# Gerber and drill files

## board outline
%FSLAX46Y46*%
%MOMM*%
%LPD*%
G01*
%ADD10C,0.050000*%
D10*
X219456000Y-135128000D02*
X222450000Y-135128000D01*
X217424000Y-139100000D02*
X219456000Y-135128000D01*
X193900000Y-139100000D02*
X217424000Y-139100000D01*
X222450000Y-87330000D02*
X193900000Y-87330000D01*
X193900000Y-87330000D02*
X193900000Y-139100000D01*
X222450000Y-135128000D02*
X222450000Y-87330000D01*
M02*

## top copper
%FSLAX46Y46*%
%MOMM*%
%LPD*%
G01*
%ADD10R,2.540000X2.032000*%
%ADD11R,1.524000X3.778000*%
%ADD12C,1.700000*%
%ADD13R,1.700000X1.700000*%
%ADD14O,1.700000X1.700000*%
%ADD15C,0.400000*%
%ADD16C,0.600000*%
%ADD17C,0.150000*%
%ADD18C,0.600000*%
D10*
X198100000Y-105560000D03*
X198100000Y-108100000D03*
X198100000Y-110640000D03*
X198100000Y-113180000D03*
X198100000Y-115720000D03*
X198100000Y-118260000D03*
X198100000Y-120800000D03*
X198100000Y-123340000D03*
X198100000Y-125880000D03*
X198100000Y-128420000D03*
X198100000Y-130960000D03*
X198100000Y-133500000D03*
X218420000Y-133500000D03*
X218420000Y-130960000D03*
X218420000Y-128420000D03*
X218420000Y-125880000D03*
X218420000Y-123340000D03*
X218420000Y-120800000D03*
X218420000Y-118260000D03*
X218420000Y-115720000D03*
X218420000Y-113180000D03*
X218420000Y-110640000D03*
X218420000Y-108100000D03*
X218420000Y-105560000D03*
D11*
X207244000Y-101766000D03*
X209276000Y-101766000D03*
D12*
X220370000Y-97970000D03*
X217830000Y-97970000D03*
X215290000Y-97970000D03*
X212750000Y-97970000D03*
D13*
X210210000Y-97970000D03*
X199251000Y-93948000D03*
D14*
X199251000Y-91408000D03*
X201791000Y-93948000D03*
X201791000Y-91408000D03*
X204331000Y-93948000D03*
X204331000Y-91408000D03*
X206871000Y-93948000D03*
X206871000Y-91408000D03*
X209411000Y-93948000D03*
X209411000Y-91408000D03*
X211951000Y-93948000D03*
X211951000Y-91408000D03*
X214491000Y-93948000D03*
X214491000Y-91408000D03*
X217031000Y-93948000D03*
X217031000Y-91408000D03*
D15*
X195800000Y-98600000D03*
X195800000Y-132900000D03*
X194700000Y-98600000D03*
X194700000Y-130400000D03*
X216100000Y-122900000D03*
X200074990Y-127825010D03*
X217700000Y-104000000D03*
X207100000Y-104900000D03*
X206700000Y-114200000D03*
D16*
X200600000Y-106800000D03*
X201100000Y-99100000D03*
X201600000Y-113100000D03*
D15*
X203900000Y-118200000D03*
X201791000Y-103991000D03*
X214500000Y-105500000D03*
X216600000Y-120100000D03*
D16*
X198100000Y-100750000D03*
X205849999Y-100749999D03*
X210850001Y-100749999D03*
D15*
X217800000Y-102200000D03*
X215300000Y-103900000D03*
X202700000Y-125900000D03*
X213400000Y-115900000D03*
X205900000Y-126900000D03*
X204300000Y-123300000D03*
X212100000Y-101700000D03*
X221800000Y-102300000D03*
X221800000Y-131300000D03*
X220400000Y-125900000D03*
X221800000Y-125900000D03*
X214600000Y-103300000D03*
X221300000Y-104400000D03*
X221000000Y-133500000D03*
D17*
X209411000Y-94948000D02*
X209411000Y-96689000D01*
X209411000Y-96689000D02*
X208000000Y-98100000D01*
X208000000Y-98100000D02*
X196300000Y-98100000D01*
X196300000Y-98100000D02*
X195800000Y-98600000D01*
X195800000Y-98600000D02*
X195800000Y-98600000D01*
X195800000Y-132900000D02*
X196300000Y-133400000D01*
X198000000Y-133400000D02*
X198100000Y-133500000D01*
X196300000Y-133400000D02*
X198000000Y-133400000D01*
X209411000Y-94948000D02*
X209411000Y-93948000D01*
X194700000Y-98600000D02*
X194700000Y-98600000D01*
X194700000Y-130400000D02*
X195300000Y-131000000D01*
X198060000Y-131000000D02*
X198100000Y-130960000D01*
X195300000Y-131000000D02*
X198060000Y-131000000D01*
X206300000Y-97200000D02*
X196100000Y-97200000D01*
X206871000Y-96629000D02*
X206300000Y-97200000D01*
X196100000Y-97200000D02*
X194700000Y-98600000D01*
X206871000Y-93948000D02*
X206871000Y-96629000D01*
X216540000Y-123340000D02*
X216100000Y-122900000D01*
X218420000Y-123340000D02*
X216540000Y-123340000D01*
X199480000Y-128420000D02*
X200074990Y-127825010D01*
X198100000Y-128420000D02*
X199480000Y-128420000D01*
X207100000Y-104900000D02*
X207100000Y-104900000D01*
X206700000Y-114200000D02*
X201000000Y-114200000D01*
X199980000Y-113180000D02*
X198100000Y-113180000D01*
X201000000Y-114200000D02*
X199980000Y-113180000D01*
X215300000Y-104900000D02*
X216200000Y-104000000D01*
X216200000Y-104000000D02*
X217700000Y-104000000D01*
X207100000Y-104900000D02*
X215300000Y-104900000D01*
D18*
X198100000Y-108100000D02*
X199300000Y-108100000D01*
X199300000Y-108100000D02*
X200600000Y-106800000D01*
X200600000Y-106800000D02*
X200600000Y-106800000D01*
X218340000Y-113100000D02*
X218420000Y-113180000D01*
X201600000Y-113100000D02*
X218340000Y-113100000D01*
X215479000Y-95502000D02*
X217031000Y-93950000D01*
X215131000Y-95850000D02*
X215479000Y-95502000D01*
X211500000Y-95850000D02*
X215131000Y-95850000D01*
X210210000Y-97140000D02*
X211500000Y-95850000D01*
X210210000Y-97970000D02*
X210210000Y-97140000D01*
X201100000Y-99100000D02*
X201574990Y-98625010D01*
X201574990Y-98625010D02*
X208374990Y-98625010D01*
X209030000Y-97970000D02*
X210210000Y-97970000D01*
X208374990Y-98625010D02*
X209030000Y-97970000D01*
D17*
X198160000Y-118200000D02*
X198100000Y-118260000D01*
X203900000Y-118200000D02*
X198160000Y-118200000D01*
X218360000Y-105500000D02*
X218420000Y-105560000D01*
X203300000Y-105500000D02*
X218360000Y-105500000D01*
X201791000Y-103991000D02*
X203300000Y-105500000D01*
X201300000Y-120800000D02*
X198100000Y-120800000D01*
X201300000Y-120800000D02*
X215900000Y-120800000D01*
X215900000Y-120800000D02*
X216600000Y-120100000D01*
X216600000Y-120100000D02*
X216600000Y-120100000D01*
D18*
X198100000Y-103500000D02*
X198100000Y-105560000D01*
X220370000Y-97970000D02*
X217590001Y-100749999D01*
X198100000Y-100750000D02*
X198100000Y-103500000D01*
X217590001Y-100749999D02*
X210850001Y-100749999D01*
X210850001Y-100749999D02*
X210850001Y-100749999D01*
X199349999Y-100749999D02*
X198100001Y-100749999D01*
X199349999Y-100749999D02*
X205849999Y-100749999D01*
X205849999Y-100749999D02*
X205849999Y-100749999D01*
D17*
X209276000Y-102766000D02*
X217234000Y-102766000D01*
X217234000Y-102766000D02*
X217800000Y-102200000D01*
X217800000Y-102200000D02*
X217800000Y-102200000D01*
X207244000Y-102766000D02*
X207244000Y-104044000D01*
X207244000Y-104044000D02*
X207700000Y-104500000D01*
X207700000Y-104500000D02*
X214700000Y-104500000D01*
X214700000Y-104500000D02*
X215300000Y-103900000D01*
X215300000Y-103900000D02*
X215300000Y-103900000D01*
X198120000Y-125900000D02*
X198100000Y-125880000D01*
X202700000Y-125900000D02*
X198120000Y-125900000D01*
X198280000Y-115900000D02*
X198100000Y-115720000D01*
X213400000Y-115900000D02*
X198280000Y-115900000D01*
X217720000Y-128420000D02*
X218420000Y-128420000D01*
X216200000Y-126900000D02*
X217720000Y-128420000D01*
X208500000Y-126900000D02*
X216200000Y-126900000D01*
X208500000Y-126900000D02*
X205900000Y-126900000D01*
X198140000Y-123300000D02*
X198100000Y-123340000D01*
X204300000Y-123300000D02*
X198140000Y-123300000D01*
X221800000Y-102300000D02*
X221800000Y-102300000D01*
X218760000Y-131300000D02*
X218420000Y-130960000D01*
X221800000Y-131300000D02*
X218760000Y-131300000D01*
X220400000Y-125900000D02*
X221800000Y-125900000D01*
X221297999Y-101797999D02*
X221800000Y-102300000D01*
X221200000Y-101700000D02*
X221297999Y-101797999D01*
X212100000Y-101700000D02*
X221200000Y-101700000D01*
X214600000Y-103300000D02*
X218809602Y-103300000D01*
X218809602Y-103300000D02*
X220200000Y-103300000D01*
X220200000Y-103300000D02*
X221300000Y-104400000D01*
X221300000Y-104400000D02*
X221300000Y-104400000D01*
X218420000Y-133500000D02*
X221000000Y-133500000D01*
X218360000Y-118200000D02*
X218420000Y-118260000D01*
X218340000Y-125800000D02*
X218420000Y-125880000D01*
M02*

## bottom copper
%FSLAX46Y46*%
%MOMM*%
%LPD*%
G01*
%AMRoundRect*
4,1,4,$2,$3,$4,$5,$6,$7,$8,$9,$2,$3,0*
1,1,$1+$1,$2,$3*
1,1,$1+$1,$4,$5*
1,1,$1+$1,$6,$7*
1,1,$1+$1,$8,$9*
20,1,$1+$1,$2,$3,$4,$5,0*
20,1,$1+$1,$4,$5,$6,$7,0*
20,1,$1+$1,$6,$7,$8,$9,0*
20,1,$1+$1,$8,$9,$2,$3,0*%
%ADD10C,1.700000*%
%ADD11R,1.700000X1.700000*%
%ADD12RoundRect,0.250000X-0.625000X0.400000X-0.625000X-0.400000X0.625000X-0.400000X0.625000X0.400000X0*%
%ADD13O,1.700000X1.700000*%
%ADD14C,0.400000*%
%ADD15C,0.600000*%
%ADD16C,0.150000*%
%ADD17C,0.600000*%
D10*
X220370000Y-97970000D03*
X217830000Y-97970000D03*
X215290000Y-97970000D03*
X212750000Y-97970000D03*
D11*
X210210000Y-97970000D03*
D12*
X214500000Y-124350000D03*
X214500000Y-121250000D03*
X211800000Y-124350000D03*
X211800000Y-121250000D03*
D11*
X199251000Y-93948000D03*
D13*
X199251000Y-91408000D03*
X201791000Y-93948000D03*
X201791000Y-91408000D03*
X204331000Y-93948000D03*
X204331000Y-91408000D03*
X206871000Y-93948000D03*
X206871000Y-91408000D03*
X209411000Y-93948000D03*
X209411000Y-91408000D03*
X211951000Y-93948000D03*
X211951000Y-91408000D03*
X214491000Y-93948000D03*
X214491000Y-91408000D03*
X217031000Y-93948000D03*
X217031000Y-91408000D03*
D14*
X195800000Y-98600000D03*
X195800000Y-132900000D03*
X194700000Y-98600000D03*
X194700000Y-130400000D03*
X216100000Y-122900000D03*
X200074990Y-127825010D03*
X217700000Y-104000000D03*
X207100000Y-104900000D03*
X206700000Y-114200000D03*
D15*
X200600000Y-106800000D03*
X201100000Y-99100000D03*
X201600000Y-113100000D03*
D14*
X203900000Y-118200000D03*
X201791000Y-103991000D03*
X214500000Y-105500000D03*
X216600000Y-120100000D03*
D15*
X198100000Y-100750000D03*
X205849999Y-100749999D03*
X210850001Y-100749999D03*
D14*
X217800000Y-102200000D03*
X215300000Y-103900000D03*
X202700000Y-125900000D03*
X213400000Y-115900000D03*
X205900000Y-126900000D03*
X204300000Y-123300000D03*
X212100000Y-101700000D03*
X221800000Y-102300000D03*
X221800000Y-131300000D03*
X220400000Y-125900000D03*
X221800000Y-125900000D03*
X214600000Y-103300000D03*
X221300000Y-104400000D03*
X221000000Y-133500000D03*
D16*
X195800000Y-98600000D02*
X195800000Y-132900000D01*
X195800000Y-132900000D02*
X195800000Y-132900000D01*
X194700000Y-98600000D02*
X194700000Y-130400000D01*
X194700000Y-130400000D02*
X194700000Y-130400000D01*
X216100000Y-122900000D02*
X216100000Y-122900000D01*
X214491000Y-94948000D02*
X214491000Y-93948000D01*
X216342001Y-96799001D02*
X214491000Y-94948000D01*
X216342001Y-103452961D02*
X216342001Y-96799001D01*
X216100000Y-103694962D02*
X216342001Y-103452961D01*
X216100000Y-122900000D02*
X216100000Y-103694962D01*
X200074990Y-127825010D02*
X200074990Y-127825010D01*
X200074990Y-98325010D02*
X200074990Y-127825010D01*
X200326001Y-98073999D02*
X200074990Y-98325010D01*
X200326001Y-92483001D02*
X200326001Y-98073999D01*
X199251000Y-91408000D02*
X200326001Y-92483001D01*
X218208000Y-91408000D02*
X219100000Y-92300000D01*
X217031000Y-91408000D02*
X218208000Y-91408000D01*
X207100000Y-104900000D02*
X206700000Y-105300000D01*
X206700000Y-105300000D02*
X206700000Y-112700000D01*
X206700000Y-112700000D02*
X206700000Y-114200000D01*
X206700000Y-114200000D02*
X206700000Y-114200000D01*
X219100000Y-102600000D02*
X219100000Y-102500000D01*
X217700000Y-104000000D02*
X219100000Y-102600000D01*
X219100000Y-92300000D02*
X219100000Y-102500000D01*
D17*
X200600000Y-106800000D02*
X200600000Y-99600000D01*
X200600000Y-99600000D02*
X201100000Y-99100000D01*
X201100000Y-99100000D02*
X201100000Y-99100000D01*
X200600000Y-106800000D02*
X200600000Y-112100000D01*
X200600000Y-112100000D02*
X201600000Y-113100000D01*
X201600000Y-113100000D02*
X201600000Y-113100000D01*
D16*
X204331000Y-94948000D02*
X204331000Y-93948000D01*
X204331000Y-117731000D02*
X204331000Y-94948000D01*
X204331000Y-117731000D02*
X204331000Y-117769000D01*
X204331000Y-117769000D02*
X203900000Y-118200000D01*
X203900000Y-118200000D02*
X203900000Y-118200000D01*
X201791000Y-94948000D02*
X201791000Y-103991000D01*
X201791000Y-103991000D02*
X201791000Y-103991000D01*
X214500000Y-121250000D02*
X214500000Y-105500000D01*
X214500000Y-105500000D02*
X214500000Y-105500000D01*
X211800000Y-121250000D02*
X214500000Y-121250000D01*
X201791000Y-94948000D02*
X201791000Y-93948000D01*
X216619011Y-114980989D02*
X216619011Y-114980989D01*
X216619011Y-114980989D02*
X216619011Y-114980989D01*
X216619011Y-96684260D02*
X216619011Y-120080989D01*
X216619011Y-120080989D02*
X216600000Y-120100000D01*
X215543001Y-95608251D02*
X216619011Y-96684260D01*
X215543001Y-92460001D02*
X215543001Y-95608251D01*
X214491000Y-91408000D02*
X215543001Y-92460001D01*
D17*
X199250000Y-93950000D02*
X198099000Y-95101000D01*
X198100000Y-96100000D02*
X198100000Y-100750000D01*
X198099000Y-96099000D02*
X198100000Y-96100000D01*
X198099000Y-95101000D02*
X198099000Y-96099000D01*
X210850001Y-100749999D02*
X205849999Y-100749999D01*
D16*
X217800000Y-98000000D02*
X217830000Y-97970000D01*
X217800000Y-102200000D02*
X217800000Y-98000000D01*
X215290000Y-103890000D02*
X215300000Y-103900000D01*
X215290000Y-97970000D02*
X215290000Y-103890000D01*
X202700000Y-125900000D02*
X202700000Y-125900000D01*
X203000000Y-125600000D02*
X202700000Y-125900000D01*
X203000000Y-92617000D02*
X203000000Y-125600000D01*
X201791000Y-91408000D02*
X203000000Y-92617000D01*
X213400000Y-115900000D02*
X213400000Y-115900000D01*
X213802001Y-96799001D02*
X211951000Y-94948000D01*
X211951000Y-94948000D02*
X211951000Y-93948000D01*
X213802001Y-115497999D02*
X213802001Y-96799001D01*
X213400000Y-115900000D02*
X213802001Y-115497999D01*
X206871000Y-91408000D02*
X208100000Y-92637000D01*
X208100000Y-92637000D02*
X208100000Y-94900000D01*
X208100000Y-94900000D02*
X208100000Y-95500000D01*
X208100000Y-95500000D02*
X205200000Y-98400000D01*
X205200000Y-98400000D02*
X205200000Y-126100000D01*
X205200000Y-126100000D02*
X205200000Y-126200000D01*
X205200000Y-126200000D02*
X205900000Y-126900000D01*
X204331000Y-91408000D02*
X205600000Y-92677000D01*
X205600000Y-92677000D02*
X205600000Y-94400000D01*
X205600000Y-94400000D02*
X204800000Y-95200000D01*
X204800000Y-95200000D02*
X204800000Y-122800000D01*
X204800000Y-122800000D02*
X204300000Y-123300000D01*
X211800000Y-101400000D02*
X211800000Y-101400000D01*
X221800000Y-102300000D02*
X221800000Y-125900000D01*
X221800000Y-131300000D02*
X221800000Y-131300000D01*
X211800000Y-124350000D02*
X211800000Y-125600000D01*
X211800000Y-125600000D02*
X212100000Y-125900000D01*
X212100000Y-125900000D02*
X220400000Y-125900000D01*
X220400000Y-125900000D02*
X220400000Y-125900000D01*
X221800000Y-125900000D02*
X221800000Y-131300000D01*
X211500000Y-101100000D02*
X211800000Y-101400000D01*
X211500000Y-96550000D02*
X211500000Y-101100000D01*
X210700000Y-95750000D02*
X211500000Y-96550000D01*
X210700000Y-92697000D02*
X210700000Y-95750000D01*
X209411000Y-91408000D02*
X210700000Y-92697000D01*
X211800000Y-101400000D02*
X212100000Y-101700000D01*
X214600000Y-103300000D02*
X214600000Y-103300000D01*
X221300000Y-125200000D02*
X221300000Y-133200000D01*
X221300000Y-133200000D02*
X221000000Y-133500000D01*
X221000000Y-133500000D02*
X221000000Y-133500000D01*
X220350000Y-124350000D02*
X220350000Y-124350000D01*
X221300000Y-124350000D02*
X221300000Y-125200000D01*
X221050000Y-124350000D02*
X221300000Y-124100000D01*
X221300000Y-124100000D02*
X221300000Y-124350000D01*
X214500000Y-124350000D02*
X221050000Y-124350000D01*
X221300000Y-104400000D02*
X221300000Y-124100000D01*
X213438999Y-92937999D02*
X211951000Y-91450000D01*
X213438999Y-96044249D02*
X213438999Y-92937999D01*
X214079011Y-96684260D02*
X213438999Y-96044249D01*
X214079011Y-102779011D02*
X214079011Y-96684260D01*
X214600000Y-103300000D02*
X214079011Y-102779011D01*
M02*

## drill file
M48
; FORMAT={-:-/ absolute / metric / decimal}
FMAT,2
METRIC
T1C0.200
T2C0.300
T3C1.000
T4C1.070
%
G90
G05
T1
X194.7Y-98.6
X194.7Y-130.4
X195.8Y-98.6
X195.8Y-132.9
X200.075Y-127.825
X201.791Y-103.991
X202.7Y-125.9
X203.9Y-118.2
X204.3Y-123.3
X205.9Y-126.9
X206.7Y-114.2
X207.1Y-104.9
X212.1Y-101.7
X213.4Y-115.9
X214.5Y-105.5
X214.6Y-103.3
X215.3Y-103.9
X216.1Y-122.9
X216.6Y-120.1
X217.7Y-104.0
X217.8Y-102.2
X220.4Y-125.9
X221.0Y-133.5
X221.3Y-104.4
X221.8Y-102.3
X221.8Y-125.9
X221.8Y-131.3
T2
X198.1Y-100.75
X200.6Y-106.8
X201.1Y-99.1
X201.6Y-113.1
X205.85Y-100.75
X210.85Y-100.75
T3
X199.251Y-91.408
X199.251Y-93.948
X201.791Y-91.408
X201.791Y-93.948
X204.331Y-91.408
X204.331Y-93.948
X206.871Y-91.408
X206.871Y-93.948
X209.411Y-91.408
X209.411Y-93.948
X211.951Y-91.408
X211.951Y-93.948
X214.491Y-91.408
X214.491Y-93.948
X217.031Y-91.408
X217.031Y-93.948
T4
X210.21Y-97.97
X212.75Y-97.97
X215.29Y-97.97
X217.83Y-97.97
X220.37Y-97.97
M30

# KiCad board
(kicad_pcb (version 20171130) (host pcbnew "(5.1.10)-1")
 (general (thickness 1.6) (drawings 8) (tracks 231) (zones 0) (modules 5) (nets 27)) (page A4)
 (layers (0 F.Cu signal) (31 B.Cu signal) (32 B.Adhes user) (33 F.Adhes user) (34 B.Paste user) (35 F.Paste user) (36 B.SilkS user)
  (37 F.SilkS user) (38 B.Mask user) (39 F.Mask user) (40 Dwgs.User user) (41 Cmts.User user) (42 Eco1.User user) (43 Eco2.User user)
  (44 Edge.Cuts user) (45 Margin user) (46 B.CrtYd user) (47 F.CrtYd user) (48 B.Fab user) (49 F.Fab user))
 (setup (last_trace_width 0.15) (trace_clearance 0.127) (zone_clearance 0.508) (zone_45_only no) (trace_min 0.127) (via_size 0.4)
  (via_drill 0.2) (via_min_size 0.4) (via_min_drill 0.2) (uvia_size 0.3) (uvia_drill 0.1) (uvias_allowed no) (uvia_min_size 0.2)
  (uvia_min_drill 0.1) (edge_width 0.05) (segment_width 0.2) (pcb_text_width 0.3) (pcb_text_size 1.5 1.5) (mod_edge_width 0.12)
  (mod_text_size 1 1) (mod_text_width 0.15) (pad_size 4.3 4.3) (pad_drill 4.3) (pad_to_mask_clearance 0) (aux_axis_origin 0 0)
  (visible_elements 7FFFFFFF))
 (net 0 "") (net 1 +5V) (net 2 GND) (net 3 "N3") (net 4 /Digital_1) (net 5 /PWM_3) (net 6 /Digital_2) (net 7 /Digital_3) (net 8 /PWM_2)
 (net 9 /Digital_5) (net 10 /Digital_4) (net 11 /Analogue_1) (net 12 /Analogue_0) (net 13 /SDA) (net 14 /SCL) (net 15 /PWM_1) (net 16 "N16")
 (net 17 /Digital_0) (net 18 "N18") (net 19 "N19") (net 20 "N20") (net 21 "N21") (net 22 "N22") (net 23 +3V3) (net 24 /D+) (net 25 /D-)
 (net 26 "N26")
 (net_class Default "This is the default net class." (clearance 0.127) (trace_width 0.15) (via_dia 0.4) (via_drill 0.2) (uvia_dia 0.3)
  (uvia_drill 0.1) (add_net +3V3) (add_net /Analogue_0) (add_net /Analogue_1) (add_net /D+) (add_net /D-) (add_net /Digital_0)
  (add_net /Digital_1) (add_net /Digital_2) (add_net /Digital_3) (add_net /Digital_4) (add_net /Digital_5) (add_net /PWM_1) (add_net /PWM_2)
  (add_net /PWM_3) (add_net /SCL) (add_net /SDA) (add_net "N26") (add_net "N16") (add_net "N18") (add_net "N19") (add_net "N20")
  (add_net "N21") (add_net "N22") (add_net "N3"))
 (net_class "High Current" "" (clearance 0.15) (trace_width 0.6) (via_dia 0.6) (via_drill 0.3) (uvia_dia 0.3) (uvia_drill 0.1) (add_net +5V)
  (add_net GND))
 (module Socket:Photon (layer F.Cu) (at 198.1 133.5)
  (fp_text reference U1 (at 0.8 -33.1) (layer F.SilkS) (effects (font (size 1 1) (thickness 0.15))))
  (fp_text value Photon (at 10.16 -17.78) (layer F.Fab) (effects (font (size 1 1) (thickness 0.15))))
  (pad 1 smd rect (at 0 -27.94) (size 2.54 2.032) (layers F.Cu F.Paste F.Mask) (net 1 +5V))
  (pad 2 smd rect (at 0 -25.4) (size 2.54 2.032) (layers F.Cu F.Paste F.Mask) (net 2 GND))
  (pad 3 smd rect (at 0 -22.86) (size 2.54 2.032) (layers F.Cu F.Paste F.Mask) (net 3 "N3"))
  (pad 4 smd rect (at 0 -20.32) (size 2.54 2.032) (layers F.Cu F.Paste F.Mask) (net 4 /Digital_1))
  (pad 5 smd rect (at 0 -17.78) (size 2.54 2.032) (layers F.Cu F.Paste F.Mask) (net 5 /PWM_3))
  (pad 6 smd rect (at 0 -15.24) (size 2.54 2.032) (layers F.Cu F.Paste F.Mask) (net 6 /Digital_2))
  (pad 7 smd rect (at 0 -12.7) (size 2.54 2.032) (layers F.Cu F.Paste F.Mask) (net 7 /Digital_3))
  (pad 8 smd rect (at 0 -10.16) (size 2.54 2.032) (layers F.Cu F.Paste F.Mask) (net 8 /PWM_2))
  (pad 9 smd rect (at 0 -7.62) (size 2.54 2.032) (layers F.Cu F.Paste F.Mask) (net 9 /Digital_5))
  (pad 10 smd rect (at 0 -5.08) (size 2.54 2.032) (layers F.Cu F.Paste F.Mask) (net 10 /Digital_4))
  (pad 11 smd rect (at 0 -2.54) (size 2.54 2.032) (layers F.Cu F.Paste F.Mask) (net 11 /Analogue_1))
  (pad 12 smd rect (at 0 0) (size 2.54 2.032) (layers F.Cu F.Paste F.Mask) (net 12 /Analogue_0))
  (pad 13 smd rect (at 20.32 0) (size 2.54 2.032) (layers F.Cu F.Paste F.Mask) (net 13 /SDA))
  (pad 14 smd rect (at 20.32 -2.54) (size 2.54 2.032) (layers F.Cu F.Paste F.Mask) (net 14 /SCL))
  (pad 15 smd rect (at 20.32 -5.08) (size 2.54 2.032) (layers F.Cu F.Paste F.Mask) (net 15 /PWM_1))
  (pad 16 smd rect (at 20.32 -7.62) (size 2.54 2.032) (layers F.Cu F.Paste F.Mask) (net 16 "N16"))
  (pad 17 smd rect (at 20.32 -10.16) (size 2.54 2.032) (layers F.Cu F.Paste F.Mask) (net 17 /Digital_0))
  (pad 18 smd rect (at 20.32 -12.7) (size 2.54 2.032) (layers F.Cu F.Paste F.Mask) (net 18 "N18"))
  (pad 19 smd rect (at 20.32 -15.24) (size 2.54 2.032) (layers F.Cu F.Paste F.Mask) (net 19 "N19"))
  (pad 20 smd rect (at 20.32 -17.78) (size 2.54 2.032) (layers F.Cu F.Paste F.Mask) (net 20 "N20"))
  (pad 21 smd rect (at 20.32 -20.32) (size 2.54 2.032) (layers F.Cu F.Paste F.Mask) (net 2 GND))
  (pad 22 smd rect (at 20.32 -22.86) (size 2.54 2.032) (layers F.Cu F.Paste F.Mask) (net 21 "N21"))
  (pad 23 smd rect (at 20.32 -25.4) (size 2.54 2.032) (layers F.Cu F.Paste F.Mask) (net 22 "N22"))
  (pad 24 smd rect (at 20.32 -27.94) (size 2.54 2.032) (layers F.Cu F.Paste F.Mask) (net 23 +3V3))
  (pad 31 smd rect (at 9.144 -31.734) (size 1.524 3.778) (layers F.Cu F.Paste F.Mask) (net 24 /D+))
  (pad 30 smd rect (at 11.176 -31.734) (size 1.524 3.778) (layers F.Cu F.Paste F.Mask) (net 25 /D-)))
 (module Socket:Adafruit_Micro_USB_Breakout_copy (layer B.Cu) (at 206.4 96.7)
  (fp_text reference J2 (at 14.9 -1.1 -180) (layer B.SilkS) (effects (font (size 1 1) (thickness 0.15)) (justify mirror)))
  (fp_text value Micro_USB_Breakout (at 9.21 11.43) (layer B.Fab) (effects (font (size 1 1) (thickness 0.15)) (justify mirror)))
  (pad 5 thru_hole circle (at 13.97 1.27) (size 1.7 1.7) (drill 1.07) (layers *.Cu *.Mask) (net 1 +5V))
  (pad 4 thru_hole circle (at 11.43 1.27) (size 1.7 1.7) (drill 1.07) (layers *.Cu *.Mask) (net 25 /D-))
  (pad 3 thru_hole circle (at 8.89 1.27) (size 1.7 1.7) (drill 1.07) (layers *.Cu *.Mask) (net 24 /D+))
  (pad 2 thru_hole circle (at 6.35 1.27) (size 1.7 1.7) (drill 1.07) (layers *.Cu *.Mask) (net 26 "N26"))
  (pad 1 thru_hole rect (at 3.81 1.27) (size 1.7 1.7) (drill 1.07) (layers *.Cu *.Mask) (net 2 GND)))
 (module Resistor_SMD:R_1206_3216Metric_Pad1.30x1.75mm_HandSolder (layer B.Cu) (at 214.5 122.8 270)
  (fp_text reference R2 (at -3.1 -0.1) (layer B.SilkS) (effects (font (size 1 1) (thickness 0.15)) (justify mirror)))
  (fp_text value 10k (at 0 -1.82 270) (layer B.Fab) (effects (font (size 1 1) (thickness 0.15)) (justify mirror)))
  (pad 2 smd roundrect (at 1.55 0 270) (size 1.3 1.75) (layers B.Cu B.Paste B.Mask) (roundrect_rratio 0.192308) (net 13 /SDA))
  (pad 1 smd roundrect (at -1.55 0 270) (size 1.3 1.75) (layers B.Cu B.Paste B.Mask) (roundrect_rratio 0.192308) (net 23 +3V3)))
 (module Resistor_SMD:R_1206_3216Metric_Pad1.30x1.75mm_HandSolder (layer B.Cu) (at 211.8 122.8 270)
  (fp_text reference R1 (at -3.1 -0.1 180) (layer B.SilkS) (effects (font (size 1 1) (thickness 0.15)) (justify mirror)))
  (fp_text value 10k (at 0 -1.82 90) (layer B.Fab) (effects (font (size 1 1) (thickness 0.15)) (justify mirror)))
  (pad 2 smd roundrect (at 1.55 0 270) (size 1.3 1.75) (layers B.Cu B.Paste B.Mask) (roundrect_rratio 0.192308) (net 14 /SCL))
  (pad 1 smd roundrect (at -1.55 0 270) (size 1.3 1.75) (layers B.Cu B.Paste B.Mask) (roundrect_rratio 0.192308) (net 23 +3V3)))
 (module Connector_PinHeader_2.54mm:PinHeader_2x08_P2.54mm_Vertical (layer F.Cu) (at 199.251 93.948 90)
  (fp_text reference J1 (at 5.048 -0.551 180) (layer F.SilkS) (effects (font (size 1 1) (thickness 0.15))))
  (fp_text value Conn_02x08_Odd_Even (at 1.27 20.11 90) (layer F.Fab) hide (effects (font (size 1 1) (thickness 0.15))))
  (pad 1 thru_hole rect (at 0 0 90) (size 1.7 1.7) (drill 1) (layers *.Cu *.Mask) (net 1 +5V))
  (pad 2 thru_hole oval (at 2.54 0 90) (size 1.7 1.7) (drill 1) (layers *.Cu *.Mask) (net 10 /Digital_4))
  (pad 3 thru_hole oval (at 0 2.54 90) (size 1.7 1.7) (drill 1) (layers *.Cu *.Mask) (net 23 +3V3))
  (pad 4 thru_hole oval (at 2.54 2.54 90) (size 1.7 1.7) (drill 1) (layers *.Cu *.Mask) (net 9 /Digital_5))
  (pad 5 thru_hole oval (at 0 5.08 90) (size 1.7 1.7) (drill 1) (layers *.Cu *.Mask) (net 6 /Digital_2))
  (pad 6 thru_hole oval (at 2.54 5.08 90) (size 1.7 1.7) (drill 1) (layers *.Cu *.Mask) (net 8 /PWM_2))
  (pad 7 thru_hole oval (at 0 7.62 90) (size 1.7 1.7) (drill 1) (layers *.Cu *.Mask) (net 11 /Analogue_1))
  (pad 8 thru_hole oval (at 2.54 7.62 90) (size 1.7 1.7) (drill 1) (layers *.Cu *.Mask) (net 15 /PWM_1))
  (pad 9 thru_hole oval (at 0 10.16 90) (size 1.7 1.7) (drill 1) (layers *.Cu *.Mask) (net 12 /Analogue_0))
  (pad 10 thru_hole oval (at 2.54 10.16 90) (size 1.7 1.7) (drill 1) (layers *.Cu *.Mask) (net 14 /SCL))
  (pad 11 thru_hole oval (at 0 12.7 90) (size 1.7 1.7) (drill 1) (layers *.Cu *.Mask) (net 5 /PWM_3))
  (pad 12 thru_hole oval (at 2.54 12.7 90) (size 1.7 1.7) (drill 1) (layers *.Cu *.Mask) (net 13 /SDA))
  (pad 13 thru_hole oval (at 0 15.24 90) (size 1.7 1.7) (drill 1) (layers *.Cu *.Mask) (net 17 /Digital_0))
  (pad 14 thru_hole oval (at 2.54 15.24 90) (size 1.7 1.7) (drill 1) (layers *.Cu *.Mask) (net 7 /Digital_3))
  (pad 15 thru_hole oval (at 0 17.78 90) (size 1.7 1.7) (drill 1) (layers *.Cu *.Mask) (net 2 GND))
  (pad 16 thru_hole oval (at 2.54 17.78 90) (size 1.7 1.7) (drill 1) (layers *.Cu *.Mask) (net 4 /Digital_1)))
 (gr_line (start 219.456 135.128) (end 222.45 135.128) (layer Edge.Cuts) (width 0.05))
 (gr_line (start 217.424 139.1) (end 219.456 135.128) (layer Edge.Cuts) (width 0.05))
 (gr_line (start 193.9 139.1) (end 217.424 139.1) (layer Edge.Cuts) (width 0.05))
 (gr_line (start 222.45 87.33) (end 193.9 87.33) (layer Edge.Cuts) (width 0.05))
 (gr_line (start 193.9 87.33) (end 193.9 139.1) (layer Edge.Cuts) (width 0.05))
 (gr_line (start 222.45 135.128) (end 222.45 87.33) (layer Edge.Cuts) (width 0.05))
 (segment (start 209.411 94.948) (end 209.411 96.689) (width 0.15) (layer F.Cu) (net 12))
 (segment (start 209.411 96.689) (end 208 98.1) (width 0.15) (layer F.Cu) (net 12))
 (segment (start 208 98.1) (end 196.3 98.1) (width 0.15) (layer F.Cu) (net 12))
 (segment (start 196.3 98.1) (end 195.8 98.6) (width 0.15) (layer F.Cu) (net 12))
 (segment (start 195.8 98.6) (end 195.8 98.6) (width 0.15) (layer F.Cu) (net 12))
 (via (at 195.8 98.6) (size 0.4) (drill 0.2) (layers F.Cu B.Cu) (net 12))
 (segment (start 195.8 98.6) (end 195.8 132.9) (width 0.15) (layer B.Cu) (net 12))
 (segment (start 195.8 132.9) (end 195.8 132.9) (width 0.15) (layer B.Cu) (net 12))
 (via (at 195.8 132.9) (size 0.4) (drill 0.2) (layers F.Cu B.Cu) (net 12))
 (segment (start 195.8 132.9) (end 196.3 133.4) (width 0.15) (layer F.Cu) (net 12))
 (segment (start 198 133.4) (end 198.1 133.5) (width 0.15) (layer F.Cu) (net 12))
 (segment (start 196.3 133.4) (end 198 133.4) (width 0.15) (layer F.Cu) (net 12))
 (segment (start 209.411 94.948) (end 209.411 93.948) (width 0.15) (layer F.Cu) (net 12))
 (segment (start 194.7 98.6) (end 194.7 98.6) (width 0.15) (layer F.Cu) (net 11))
 (via (at 194.7 98.6) (size 0.4) (drill 0.2) (layers F.Cu B.Cu) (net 11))
 (segment (start 194.7 98.6) (end 194.7 130.4) (width 0.15) (layer B.Cu) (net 11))
 (segment (start 194.7 130.4) (end 194.7 130.4) (width 0.15) (layer B.Cu) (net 11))
 (via (at 194.7 130.4) (size 0.4) (drill 0.2) (layers F.Cu B.Cu) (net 11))
 (segment (start 194.7 130.4) (end 195.3 131) (width 0.15) (layer F.Cu) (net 11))
 (segment (start 198.06 131) (end 198.1 130.96) (width 0.15) (layer F.Cu) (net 11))
 (segment (start 195.3 131) (end 198.06 131) (width 0.15) (layer F.Cu) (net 11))
 (segment (start 206.3 97.2) (end 196.1 97.2) (width 0.15) (layer F.Cu) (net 11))
 (segment (start 206.871 96.629) (end 206.3 97.2) (width 0.15) (layer F.Cu) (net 11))
 (segment (start 196.1 97.2) (end 194.7 98.6) (width 0.15) (layer F.Cu) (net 11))
 (segment (start 206.871 93.948) (end 206.871 96.629) (width 0.15) (layer F.Cu) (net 11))
 (segment (start 216.1 122.9) (end 216.1 122.9) (width 0.15) (layer B.Cu) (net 17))
 (via (at 216.1 122.9) (size 0.4) (drill 0.2) (layers F.Cu B.Cu) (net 17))
 (segment (start 216.54 123.34) (end 216.1 122.9) (width 0.15) (layer F.Cu) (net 17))
 (segment (start 218.42 123.34) (end 216.54 123.34) (width 0.15) (layer F.Cu) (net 17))
 (segment (start 214.491 94.948) (end 214.491 93.948) (width 0.15) (layer B.Cu) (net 17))
 (segment (start 216.342001 96.799001) (end 214.491 94.948) (width 0.15) (layer B.Cu) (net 17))
 (segment (start 216.342001 103.452961) (end 216.342001 96.799001) (width 0.15) (layer B.Cu) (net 17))
 (segment (start 216.1 103.694962) (end 216.342001 103.452961) (width 0.15) (layer B.Cu) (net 17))
 (segment (start 216.1 122.9) (end 216.1 103.694962) (width 0.15) (layer B.Cu) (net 17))
 (segment (start 200.07499 127.82501) (end 200.07499 127.82501) (width 0.15) (layer B.Cu) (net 10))
 (via (at 200.07499 127.82501) (size 0.4) (drill 0.2) (layers F.Cu B.Cu) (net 10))
 (segment (start 199.48 128.42) (end 200.07499 127.82501) (width 0.15) (layer F.Cu) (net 10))
 (segment (start 198.1 128.42) (end 199.48 128.42) (width 0.15) (layer F.Cu) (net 10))
 (segment (start 200.07499 98.32501) (end 200.07499 127.82501) (width 0.15) (layer B.Cu) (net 10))
 (segment (start 200.326001 98.073999) (end 200.07499 98.32501) (width 0.15) (layer B.Cu) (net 10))
 (segment (start 200.326001 92.483001) (end 200.326001 98.073999) (width 0.15) (layer B.Cu) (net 10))
 (segment (start 199.251 91.408) (end 200.326001 92.483001) (width 0.15) (layer B.Cu) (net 10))
 (segment (start 218.208 91.408) (end 219.1 92.3) (width 0.15) (layer B.Cu) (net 4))
 (segment (start 217.031 91.408) (end 218.208 91.408) (width 0.15) (layer B.Cu) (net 4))
 (via (at 217.7 104) (size 0.4) (drill 0.2) (layers F.Cu B.Cu) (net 4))
 (segment (start 207.1 104.9) (end 207.1 104.9) (width 0.15) (layer F.Cu) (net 4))
 (via (at 207.1 104.9) (size 0.4) (drill 0.2) (layers F.Cu B.Cu) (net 4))
 (segment (start 207.1 104.9) (end 206.7 105.3) (width 0.15) (layer B.Cu) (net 4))
 (segment (start 206.7 105.3) (end 206.7 112.7) (width 0.15) (layer B.Cu) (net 4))
 (segment (start 206.7 112.7) (end 206.7 114.2) (width 0.15) (layer B.Cu) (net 4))
 (segment (start 206.7 114.2) (end 206.7 114.2) (width 0.15) (layer B.Cu) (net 4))
 (via (at 206.7 114.2) (size 0.4) (drill 0.2) (layers F.Cu B.Cu) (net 4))
 (segment (start 206.7 114.2) (end 201 114.2) (width 0.15) (layer F.Cu) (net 4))
 (segment (start 199.98 113.18) (end 198.1 113.18) (width 0.15) (layer F.Cu) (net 4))
 (segment (start 201 114.2) (end 199.98 113.18) (width 0.15) (layer F.Cu) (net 4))
 (segment (start 219.1 102.6) (end 219.1 102.5) (width 0.15) (layer B.Cu) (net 4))
 (segment (start 217.7 104) (end 219.1 102.6) (width 0.15) (layer B.Cu) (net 4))
 (segment (start 219.1 92.3) (end 219.1 102.5) (width 0.15) (layer B.Cu) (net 4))
 (segment (start 215.3 104.9) (end 216.2 104) (width 0.15) (layer F.Cu) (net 4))
 (segment (start 216.2 104) (end 217.7 104) (width 0.15) (layer F.Cu) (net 4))
 (segment (start 207.1 104.9) (end 215.3 104.9) (width 0.15) (layer F.Cu) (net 4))
 (segment (start 198.1 108.1) (end 199.3 108.1) (width 0.6) (layer F.Cu) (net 2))
 (segment (start 199.3 108.1) (end 200.6 106.8) (width 0.6) (layer F.Cu) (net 2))
 (segment (start 200.6 106.8) (end 200.6 106.8) (width 0.6) (layer F.Cu) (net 2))
 (via (at 200.6 106.8) (size 0.6) (drill 0.3) (layers F.Cu B.Cu) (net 2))
 (segment (start 200.6 106.8) (end 200.6 99.6) (width 0.6) (layer B.Cu) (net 2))
 (segment (start 200.6 99.6) (end 201.1 99.1) (width 0.6) (layer B.Cu) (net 2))
 (segment (start 201.1 99.1) (end 201.1 99.1) (width 0.6) (layer B.Cu) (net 2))
 (via (at 201.1 99.1) (size 0.6) (drill 0.3) (layers F.Cu B.Cu) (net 2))
 (segment (start 200.6 106.8) (end 200.6 112.1) (width 0.6) (layer B.Cu) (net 2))
 (segment (start 200.6 112.1) (end 201.6 113.1) (width 0.6) (layer B.Cu) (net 2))
 (segment (start 201.6 113.1) (end 201.6 113.1) (width 0.6) (layer B.Cu) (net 2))
 (via (at 201.6 113.1) (size 0.6) (drill 0.3) (layers F.Cu B.Cu) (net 2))
 (segment (start 218.34 113.1) (end 218.42 113.18) (width 0.6) (layer F.Cu) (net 2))
 (segment (start 201.6 113.1) (end 218.34 113.1) (width 0.6) (layer F.Cu) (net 2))
 (segment (start 215.479 95.502) (end 217.031 93.95) (width 0.6) (layer F.Cu) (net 2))
 (segment (start 215.131 95.85) (end 215.479 95.502) (width 0.6) (layer F.Cu) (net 2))
 (segment (start 211.5 95.85) (end 215.131 95.85) (width 0.6) (layer F.Cu) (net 2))
 (segment (start 210.21 97.14) (end 211.5 95.85) (width 0.6) (layer F.Cu) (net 2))
 (segment (start 210.21 97.97) (end 210.21 97.14) (width 0.6) (layer F.Cu) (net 2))
 (segment (start 201.1 99.1) (end 201.57499 98.62501) (width 0.6) (layer F.Cu) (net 2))
 (segment (start 201.57499 98.62501) (end 208.37499 98.62501) (width 0.6) (layer F.Cu) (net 2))
 (segment (start 209.03 97.97) (end 210.21 97.97) (width 0.6) (layer F.Cu) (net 2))
 (segment (start 208.37499 98.62501) (end 209.03 97.97) (width 0.6) (layer F.Cu) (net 2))
 (segment (start 204.331 94.948) (end 204.331 93.948) (width 0.15) (layer B.Cu) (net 6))
 (segment (start 204.331 117.731) (end 204.331 94.948) (width 0.15) (layer B.Cu) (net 6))
 (segment (start 204.331 117.731) (end 204.331 117.769) (width 0.15) (layer B.Cu) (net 6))
 (segment (start 204.331 117.769) (end 203.9 118.2) (width 0.15) (layer B.Cu) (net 6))
 (segment (start 203.9 118.2) (end 203.9 118.2) (width 0.15) (layer B.Cu) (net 6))
 (via (at 203.9 118.2) (size 0.4) (drill 0.2) (layers F.Cu B.Cu) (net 6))
 (segment (start 198.16 118.2) (end 198.1 118.26) (width 0.15) (layer F.Cu) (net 6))
 (segment (start 203.9 118.2) (end 198.16 118.2) (width 0.15) (layer F.Cu) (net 6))
 (segment (start 201.791 94.948) (end 201.791 103.991) (width 0.15) (layer B.Cu) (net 23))
 (segment (start 218.36 105.5) (end 218.42 105.56) (width 0.15) (layer F.Cu) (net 23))
 (segment (start 203.3 105.5) (end 218.36 105.5) (width 0.15) (layer F.Cu) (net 23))
 (segment (start 201.791 103.991) (end 201.791 103.991) (width 0.15) (layer B.Cu) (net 23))
 (via (at 201.791 103.991) (size 0.4) (drill 0.2) (layers F.Cu B.Cu) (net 23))
 (segment (start 201.791 103.991) (end 203.3 105.5) (width 0.15) (layer F.Cu) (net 23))
 (segment (start 214.5 121.25) (end 214.5 105.5) (width 0.15) (layer B.Cu) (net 23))
 (segment (start 214.5 105.5) (end 214.5 105.5) (width 0.15) (layer B.Cu) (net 23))
 (via (at 214.5 105.5) (size 0.4) (drill 0.2) (layers F.Cu B.Cu) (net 23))
 (segment (start 211.8 121.25) (end 214.5 121.25) (width 0.15) (layer B.Cu) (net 23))
 (segment (start 201.791 94.948) (end 201.791 93.948) (width 0.15) (layer B.Cu) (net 23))
 (segment (start 216.619011 114.980989) (end 216.619011 114.980989) (width 0.15) (layer B.Cu) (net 7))
 (segment (start 216.619011 114.980989) (end 216.619011 114.980989) (width 0.15) (layer B.Cu) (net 7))
 (segment (start 201.3 120.8) (end 198.1 120.8) (width 0.15) (layer F.Cu) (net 7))
 (segment (start 201.3 120.8) (end 215.9 120.8) (width 0.15) (layer F.Cu) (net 7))
 (segment (start 215.9 120.8) (end 216.6 120.1) (width 0.15) (layer F.Cu) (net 7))
 (segment (start 216.6 120.1) (end 216.6 120.1) (width 0.15) (layer F.Cu) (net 7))
 (via (at 216.6 120.1) (size 0.4) (drill 0.2) (layers F.Cu B.Cu) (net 7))
 (segment (start 216.619011 96.68426) (end 216.619011 120.080989) (width 0.15) (layer B.Cu) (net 7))
 (segment (start 216.619011 120.080989) (end 216.6 120.1) (width 0.15) (layer B.Cu) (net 7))
 (segment (start 215.543001 95.608251) (end 216.619011 96.68426) (width 0.15) (layer B.Cu) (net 7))
 (segment (start 215.543001 92.460001) (end 215.543001 95.608251) (width 0.15) (layer B.Cu) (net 7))
 (segment (start 214.491 91.408) (end 215.543001 92.460001) (width 0.15) (layer B.Cu) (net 7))
 (segment (start 199.25 93.95) (end 198.099 95.101) (width 0.6) (layer B.Cu) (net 1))
 (segment (start 198.1 96.1) (end 198.1 100.75) (width 0.6) (layer B.Cu) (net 1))
 (segment (start 198.1 103.5) (end 198.1 105.56) (width 0.6) (layer F.Cu) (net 1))
 (segment (start 220.37 97.97) (end 217.590001 100.749999) (width 0.6) (layer F.Cu) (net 1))
 (via (at 198.1 100.75) (size 0.6) (drill 0.3) (layers F.Cu B.Cu) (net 1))
 (segment (start 198.099 96.099) (end 198.1 96.1) (width 0.6) (layer B.Cu) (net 1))
 (segment (start 198.099 95.101) (end 198.099 96.099) (width 0.6) (layer B.Cu) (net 1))
 (segment (start 198.1 100.75) (end 198.1 103.5) (width 0.6) (layer F.Cu) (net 1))
 (via (at 205.849999 100.749999) (size 0.6) (drill 0.3) (layers F.Cu B.Cu) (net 1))
 (segment (start 217.590001 100.749999) (end 210.850001 100.749999) (width 0.6) (layer F.Cu) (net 1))
 (segment (start 210.850001 100.749999) (end 210.850001 100.749999) (width 0.6) (layer F.Cu) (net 1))
 (via (at 210.850001 100.749999) (size 0.6) (drill 0.3) (layers F.Cu B.Cu) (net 1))
 (segment (start 199.349999 100.749999) (end 198.100001 100.749999) (width 0.6) (layer F.Cu) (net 1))
 (segment (start 199.349999 100.749999) (end 205.849999 100.749999) (width 0.6) (layer F.Cu) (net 1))
 (segment (start 205.849999 100.749999) (end 205.849999 100.749999) (width 0.6) (layer F.Cu) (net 1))
 (segment (start 210.850001 100.749999) (end 205.849999 100.749999) (width 0.6) (layer B.Cu) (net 1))
 (segment (start 209.276 102.766) (end 217.234 102.766) (width 0.15) (layer F.Cu) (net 25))
 (segment (start 217.234 102.766) (end 217.8 102.2) (width 0.15) (layer F.Cu) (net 25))
 (segment (start 217.8 102.2) (end 217.8 102.2) (width 0.15) (layer F.Cu) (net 25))
 (via (at 217.8 102.2) (size 0.4) (drill 0.2) (layers F.Cu B.Cu) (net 25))
 (segment (start 217.8 98) (end 217.83 97.97) (width 0.15) (layer B.Cu) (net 25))
 (segment (start 217.8 102.2) (end 217.8 98) (width 0.15) (layer B.Cu) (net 25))
 (segment (start 207.244 102.766) (end 207.244 104.044) (width 0.15) (layer F.Cu) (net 24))
 (segment (start 207.244 104.044) (end 207.7 104.5) (width 0.15) (layer F.Cu) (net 24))
 (segment (start 207.7 104.5) (end 214.7 104.5) (width 0.15) (layer F.Cu) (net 24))
 (segment (start 214.7 104.5) (end 215.3 103.9) (width 0.15) (layer F.Cu) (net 24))
 (segment (start 215.3 103.9) (end 215.3 103.9) (width 0.15) (layer F.Cu) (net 24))
 (via (at 215.3 103.9) (size 0.4) (drill 0.2) (layers F.Cu B.Cu) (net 24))
 (segment (start 215.29 103.89) (end 215.3 103.9) (width 0.15) (layer B.Cu) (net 24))
 (segment (start 215.29 97.97) (end 215.29 103.89) (width 0.15) (layer B.Cu) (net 24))
 (segment (start 202.7 125.9) (end 202.7 125.9) (width 0.15) (layer B.Cu) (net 9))
 (via (at 202.7 125.9) (size 0.4) (drill 0.2) (layers F.Cu B.Cu) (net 9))
 (segment (start 198.12 125.9) (end 198.1 125.88) (width 0.15) (layer F.Cu) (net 9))
 (segment (start 202.7 125.9) (end 198.12 125.9) (width 0.15) (layer F.Cu) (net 9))
 (segment (start 203 125.6) (end 202.7 125.9) (width 0.15) (layer B.Cu) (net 9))
 (segment (start 203 92.617) (end 203 125.6) (width 0.15) (layer B.Cu) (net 9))
 (segment (start 201.791 91.408) (end 203 92.617) (width 0.15) (layer B.Cu) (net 9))
 (segment (start 213.4 115.9) (end 213.4 115.9) (width 0.15) (layer B.Cu) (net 5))
 (via (at 213.4 115.9) (size 0.4) (drill 0.2) (layers F.Cu B.Cu) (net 5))
 (segment (start 198.28 115.9) (end 198.1 115.72) (width 0.15) (layer F.Cu) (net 5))
 (segment (start 213.4 115.9) (end 198.28 115.9) (width 0.15) (layer F.Cu) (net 5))
 (segment (start 213.802001 96.799001) (end 211.951 94.948) (width 0.15) (layer B.Cu) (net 5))
 (segment (start 211.951 94.948) (end 211.951 93.948) (width 0.15) (layer B.Cu) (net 5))
 (segment (start 213.802001 115.497999) (end 213.802001 96.799001) (width 0.15) (layer B.Cu) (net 5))
 (segment (start 213.4 115.9) (end 213.802001 115.497999) (width 0.15) (layer B.Cu) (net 5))
 (via (at 205.9 126.9) (size 0.4) (drill 0.2) (layers F.Cu B.Cu) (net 15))
 (segment (start 217.72 128.42) (end 218.42 128.42) (width 0.15) (layer F.Cu) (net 15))
 (segment (start 216.2 126.9) (end 217.72 128.42) (width 0.15) (layer F.Cu) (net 15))
 (segment (start 208.5 126.9) (end 216.2 126.9) (width 0.15) (layer F.Cu) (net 15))
 (segment (start 206.871 91.408) (end 208.1 92.637) (width 0.15) (layer B.Cu) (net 15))
 (segment (start 208.1 92.637) (end 208.1 94.9) (width 0.15) (layer B.Cu) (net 15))
 (segment (start 208.1 94.9) (end 208.1 95.5) (width 0.15) (layer B.Cu) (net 15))
 (segment (start 208.1 95.5) (end 205.2 98.4) (width 0.15) (layer B.Cu) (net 15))
 (segment (start 205.2 98.4) (end 205.2 126.1) (width 0.15) (layer B.Cu) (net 15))
 (segment (start 205.2 126.1) (end 205.2 126.2) (width 0.15) (layer B.Cu) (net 15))
 (segment (start 205.2 126.2) (end 205.9 126.9) (width 0.15) (layer B.Cu) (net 15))
 (segment (start 208.5 126.9) (end 205.9 126.9) (width 0.15) (layer F.Cu) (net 15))
 (segment (start 204.331 91.408) (end 205.6 92.677) (width 0.15) (layer B.Cu) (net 8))
 (via (at 204.3 123.3) (size 0.4) (drill 0.2) (layers F.Cu B.Cu) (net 8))
 (segment (start 205.6 92.677) (end 205.6 94.4) (width 0.15) (layer B.Cu) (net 8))
 (segment (start 205.6 94.4) (end 204.8 95.2) (width 0.15) (layer B.Cu) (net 8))
 (segment (start 204.8 95.2) (end 204.8 122.8) (width 0.15) (layer B.Cu) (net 8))
 (segment (start 204.8 122.8) (end 204.3 123.3) (width 0.15) (layer B.Cu) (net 8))
 (segment (start 198.14 123.3) (end 198.1 123.34) (width 0.15) (layer F.Cu) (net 8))
 (segment (start 204.3 123.3) (end 198.14 123.3) (width 0.15) (layer F.Cu) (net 8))
 (segment (start 211.8 101.4) (end 211.8 101.4) (width 0.15) (layer B.Cu) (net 14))
 (via (at 212.1 101.7) (size 0.4) (drill 0.2) (layers F.Cu B.Cu) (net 14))
 (segment (start 221.8 102.3) (end 221.8 102.3) (width 0.15) (layer F.Cu) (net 14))
 (via (at 221.8 102.3) (size 0.4) (drill 0.2) (layers F.Cu B.Cu) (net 14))
 (segment (start 221.8 102.3) (end 221.8 125.9) (width 0.15) (layer B.Cu) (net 14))
 (segment (start 221.8 131.3) (end 221.8 131.3) (width 0.15) (layer B.Cu) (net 14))
 (via (at 221.8 131.3) (size 0.4) (drill 0.2) (layers F.Cu B.Cu) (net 14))
 (segment (start 218.76 131.3) (end 218.42 130.96) (width 0.15) (layer F.Cu) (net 14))
 (segment (start 221.8 131.3) (end 218.76 131.3) (width 0.15) (layer F.Cu) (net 14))
 (segment (start 211.8 124.35) (end 211.8 125.6) (width 0.15) (layer B.Cu) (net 14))
 (segment (start 211.8 125.6) (end 212.1 125.9) (width 0.15) (layer B.Cu) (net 14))
 (segment (start 212.1 125.9) (end 220.4 125.9) (width 0.15) (layer B.Cu) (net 14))
 (segment (start 220.4 125.9) (end 220.4 125.9) (width 0.15) (layer B.Cu) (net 14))
 (via (at 220.4 125.9) (size 0.4) (drill 0.2) (layers F.Cu B.Cu) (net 14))
 (segment (start 221.8 125.9) (end 221.8 131.3) (width 0.15) (layer B.Cu) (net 14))
 (via (at 221.8 125.9) (size 0.4) (drill 0.2) (layers F.Cu B.Cu) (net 14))
 (segment (start 220.4 125.9) (end 221.8 125.9) (width 0.15) (layer F.Cu) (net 14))
 (segment (start 211.5 101.1) (end 211.8 101.4) (width 0.15) (layer B.Cu) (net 14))
 (segment (start 211.5 96.55) (end 211.5 101.1) (width 0.15) (layer B.Cu) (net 14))
 (segment (start 210.7 95.75) (end 211.5 96.55) (width 0.15) (layer B.Cu) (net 14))
 (segment (start 210.7 92.697) (end 210.7 95.75) (width 0.15) (layer B.Cu) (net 14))
 (segment (start 209.411 91.408) (end 210.7 92.697) (width 0.15) (layer B.Cu) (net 14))
 (segment (start 221.297999 101.797999) (end 221.8 102.3) (width 0.15) (layer F.Cu) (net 14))
 (segment (start 211.8 101.4) (end 212.1 101.7) (width 0.15) (layer B.Cu) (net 14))
 (segment (start 221.2 101.7) (end 221.297999 101.797999) (width 0.15) (layer F.Cu) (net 14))
 (segment (start 212.1 101.7) (end 221.2 101.7) (width 0.15) (layer F.Cu) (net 14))
 (segment (start 214.6 103.3) (end 214.6 103.3) (width 0.15) (layer B.Cu) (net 13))
 (via (at 214.6 103.3) (size 0.4) (drill 0.2) (layers F.Cu B.Cu) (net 13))
 (segment (start 214.6 103.3) (end 218.809602 103.3) (width 0.15) (layer F.Cu) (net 13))
 (segment (start 218.809602 103.3) (end 220.2 103.3) (width 0.15) (layer F.Cu) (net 13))
 (segment (start 220.2 103.3) (end 221.3 104.4) (width 0.15) (layer F.Cu) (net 13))
 (segment (start 221.3 104.4) (end 221.3 104.4) (width 0.15) (layer F.Cu) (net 13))
 (via (at 221.3 104.4) (size 0.4) (drill 0.2) (layers F.Cu B.Cu) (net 13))
 (segment (start 221.3 125.2) (end 221.3 133.2) (width 0.15) (layer B.Cu) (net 13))
 (segment (start 221.3 133.2) (end 221 133.5) (width 0.15) (layer B.Cu) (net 13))
 (segment (start 221 133.5) (end 221 133.5) (width 0.15) (layer B.Cu) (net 13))
 (via (at 221 133.5) (size 0.4) (drill 0.2) (layers F.Cu B.Cu) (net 13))
 (segment (start 218.42 133.5) (end 221 133.5) (width 0.15) (layer F.Cu) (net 13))
 (segment (start 220.35 124.35) (end 220.35 124.35) (width 0.15) (layer B.Cu) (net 13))
 (segment (start 221.3 124.35) (end 221.3 125.2) (width 0.15) (layer B.Cu) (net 13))
 (segment (start 221.05 124.35) (end 221.3 124.1) (width 0.15) (layer B.Cu) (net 13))
 (segment (start 221.3 124.1) (end 221.3 124.35) (width 0.15) (layer B.Cu) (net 13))
 (segment (start 214.5 124.35) (end 221.05 124.35) (width 0.15) (layer B.Cu) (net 13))
 (segment (start 221.3 104.4) (end 221.3 124.1) (width 0.15) (layer B.Cu) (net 13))
 (segment (start 213.438999 92.937999) (end 211.951 91.45) (width 0.15) (layer B.Cu) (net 13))
 (segment (start 213.438999 96.044249) (end 213.438999 92.937999) (width 0.15) (layer B.Cu) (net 13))
 (segment (start 214.079011 96.68426) (end 213.438999 96.044249) (width 0.15) (layer B.Cu) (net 13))
 (segment (start 214.079011 102.779011) (end 214.079011 96.68426) (width 0.15) (layer B.Cu) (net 13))
 (segment (start 214.6 103.3) (end 214.079011 102.779011) (width 0.15) (layer B.Cu) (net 13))
 (segment (start 218.36 118.2) (end 218.42 118.26) (width 0.15) (layer F.Cu) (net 19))
 (segment (start 218.34 125.8) (end 218.42 125.88) (width 0.15) (layer F.Cu) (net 16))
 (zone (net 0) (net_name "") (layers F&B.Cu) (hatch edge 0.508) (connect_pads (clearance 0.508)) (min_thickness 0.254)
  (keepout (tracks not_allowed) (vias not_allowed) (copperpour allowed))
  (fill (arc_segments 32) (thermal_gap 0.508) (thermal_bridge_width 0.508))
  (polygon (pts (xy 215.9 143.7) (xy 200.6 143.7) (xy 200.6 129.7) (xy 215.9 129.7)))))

